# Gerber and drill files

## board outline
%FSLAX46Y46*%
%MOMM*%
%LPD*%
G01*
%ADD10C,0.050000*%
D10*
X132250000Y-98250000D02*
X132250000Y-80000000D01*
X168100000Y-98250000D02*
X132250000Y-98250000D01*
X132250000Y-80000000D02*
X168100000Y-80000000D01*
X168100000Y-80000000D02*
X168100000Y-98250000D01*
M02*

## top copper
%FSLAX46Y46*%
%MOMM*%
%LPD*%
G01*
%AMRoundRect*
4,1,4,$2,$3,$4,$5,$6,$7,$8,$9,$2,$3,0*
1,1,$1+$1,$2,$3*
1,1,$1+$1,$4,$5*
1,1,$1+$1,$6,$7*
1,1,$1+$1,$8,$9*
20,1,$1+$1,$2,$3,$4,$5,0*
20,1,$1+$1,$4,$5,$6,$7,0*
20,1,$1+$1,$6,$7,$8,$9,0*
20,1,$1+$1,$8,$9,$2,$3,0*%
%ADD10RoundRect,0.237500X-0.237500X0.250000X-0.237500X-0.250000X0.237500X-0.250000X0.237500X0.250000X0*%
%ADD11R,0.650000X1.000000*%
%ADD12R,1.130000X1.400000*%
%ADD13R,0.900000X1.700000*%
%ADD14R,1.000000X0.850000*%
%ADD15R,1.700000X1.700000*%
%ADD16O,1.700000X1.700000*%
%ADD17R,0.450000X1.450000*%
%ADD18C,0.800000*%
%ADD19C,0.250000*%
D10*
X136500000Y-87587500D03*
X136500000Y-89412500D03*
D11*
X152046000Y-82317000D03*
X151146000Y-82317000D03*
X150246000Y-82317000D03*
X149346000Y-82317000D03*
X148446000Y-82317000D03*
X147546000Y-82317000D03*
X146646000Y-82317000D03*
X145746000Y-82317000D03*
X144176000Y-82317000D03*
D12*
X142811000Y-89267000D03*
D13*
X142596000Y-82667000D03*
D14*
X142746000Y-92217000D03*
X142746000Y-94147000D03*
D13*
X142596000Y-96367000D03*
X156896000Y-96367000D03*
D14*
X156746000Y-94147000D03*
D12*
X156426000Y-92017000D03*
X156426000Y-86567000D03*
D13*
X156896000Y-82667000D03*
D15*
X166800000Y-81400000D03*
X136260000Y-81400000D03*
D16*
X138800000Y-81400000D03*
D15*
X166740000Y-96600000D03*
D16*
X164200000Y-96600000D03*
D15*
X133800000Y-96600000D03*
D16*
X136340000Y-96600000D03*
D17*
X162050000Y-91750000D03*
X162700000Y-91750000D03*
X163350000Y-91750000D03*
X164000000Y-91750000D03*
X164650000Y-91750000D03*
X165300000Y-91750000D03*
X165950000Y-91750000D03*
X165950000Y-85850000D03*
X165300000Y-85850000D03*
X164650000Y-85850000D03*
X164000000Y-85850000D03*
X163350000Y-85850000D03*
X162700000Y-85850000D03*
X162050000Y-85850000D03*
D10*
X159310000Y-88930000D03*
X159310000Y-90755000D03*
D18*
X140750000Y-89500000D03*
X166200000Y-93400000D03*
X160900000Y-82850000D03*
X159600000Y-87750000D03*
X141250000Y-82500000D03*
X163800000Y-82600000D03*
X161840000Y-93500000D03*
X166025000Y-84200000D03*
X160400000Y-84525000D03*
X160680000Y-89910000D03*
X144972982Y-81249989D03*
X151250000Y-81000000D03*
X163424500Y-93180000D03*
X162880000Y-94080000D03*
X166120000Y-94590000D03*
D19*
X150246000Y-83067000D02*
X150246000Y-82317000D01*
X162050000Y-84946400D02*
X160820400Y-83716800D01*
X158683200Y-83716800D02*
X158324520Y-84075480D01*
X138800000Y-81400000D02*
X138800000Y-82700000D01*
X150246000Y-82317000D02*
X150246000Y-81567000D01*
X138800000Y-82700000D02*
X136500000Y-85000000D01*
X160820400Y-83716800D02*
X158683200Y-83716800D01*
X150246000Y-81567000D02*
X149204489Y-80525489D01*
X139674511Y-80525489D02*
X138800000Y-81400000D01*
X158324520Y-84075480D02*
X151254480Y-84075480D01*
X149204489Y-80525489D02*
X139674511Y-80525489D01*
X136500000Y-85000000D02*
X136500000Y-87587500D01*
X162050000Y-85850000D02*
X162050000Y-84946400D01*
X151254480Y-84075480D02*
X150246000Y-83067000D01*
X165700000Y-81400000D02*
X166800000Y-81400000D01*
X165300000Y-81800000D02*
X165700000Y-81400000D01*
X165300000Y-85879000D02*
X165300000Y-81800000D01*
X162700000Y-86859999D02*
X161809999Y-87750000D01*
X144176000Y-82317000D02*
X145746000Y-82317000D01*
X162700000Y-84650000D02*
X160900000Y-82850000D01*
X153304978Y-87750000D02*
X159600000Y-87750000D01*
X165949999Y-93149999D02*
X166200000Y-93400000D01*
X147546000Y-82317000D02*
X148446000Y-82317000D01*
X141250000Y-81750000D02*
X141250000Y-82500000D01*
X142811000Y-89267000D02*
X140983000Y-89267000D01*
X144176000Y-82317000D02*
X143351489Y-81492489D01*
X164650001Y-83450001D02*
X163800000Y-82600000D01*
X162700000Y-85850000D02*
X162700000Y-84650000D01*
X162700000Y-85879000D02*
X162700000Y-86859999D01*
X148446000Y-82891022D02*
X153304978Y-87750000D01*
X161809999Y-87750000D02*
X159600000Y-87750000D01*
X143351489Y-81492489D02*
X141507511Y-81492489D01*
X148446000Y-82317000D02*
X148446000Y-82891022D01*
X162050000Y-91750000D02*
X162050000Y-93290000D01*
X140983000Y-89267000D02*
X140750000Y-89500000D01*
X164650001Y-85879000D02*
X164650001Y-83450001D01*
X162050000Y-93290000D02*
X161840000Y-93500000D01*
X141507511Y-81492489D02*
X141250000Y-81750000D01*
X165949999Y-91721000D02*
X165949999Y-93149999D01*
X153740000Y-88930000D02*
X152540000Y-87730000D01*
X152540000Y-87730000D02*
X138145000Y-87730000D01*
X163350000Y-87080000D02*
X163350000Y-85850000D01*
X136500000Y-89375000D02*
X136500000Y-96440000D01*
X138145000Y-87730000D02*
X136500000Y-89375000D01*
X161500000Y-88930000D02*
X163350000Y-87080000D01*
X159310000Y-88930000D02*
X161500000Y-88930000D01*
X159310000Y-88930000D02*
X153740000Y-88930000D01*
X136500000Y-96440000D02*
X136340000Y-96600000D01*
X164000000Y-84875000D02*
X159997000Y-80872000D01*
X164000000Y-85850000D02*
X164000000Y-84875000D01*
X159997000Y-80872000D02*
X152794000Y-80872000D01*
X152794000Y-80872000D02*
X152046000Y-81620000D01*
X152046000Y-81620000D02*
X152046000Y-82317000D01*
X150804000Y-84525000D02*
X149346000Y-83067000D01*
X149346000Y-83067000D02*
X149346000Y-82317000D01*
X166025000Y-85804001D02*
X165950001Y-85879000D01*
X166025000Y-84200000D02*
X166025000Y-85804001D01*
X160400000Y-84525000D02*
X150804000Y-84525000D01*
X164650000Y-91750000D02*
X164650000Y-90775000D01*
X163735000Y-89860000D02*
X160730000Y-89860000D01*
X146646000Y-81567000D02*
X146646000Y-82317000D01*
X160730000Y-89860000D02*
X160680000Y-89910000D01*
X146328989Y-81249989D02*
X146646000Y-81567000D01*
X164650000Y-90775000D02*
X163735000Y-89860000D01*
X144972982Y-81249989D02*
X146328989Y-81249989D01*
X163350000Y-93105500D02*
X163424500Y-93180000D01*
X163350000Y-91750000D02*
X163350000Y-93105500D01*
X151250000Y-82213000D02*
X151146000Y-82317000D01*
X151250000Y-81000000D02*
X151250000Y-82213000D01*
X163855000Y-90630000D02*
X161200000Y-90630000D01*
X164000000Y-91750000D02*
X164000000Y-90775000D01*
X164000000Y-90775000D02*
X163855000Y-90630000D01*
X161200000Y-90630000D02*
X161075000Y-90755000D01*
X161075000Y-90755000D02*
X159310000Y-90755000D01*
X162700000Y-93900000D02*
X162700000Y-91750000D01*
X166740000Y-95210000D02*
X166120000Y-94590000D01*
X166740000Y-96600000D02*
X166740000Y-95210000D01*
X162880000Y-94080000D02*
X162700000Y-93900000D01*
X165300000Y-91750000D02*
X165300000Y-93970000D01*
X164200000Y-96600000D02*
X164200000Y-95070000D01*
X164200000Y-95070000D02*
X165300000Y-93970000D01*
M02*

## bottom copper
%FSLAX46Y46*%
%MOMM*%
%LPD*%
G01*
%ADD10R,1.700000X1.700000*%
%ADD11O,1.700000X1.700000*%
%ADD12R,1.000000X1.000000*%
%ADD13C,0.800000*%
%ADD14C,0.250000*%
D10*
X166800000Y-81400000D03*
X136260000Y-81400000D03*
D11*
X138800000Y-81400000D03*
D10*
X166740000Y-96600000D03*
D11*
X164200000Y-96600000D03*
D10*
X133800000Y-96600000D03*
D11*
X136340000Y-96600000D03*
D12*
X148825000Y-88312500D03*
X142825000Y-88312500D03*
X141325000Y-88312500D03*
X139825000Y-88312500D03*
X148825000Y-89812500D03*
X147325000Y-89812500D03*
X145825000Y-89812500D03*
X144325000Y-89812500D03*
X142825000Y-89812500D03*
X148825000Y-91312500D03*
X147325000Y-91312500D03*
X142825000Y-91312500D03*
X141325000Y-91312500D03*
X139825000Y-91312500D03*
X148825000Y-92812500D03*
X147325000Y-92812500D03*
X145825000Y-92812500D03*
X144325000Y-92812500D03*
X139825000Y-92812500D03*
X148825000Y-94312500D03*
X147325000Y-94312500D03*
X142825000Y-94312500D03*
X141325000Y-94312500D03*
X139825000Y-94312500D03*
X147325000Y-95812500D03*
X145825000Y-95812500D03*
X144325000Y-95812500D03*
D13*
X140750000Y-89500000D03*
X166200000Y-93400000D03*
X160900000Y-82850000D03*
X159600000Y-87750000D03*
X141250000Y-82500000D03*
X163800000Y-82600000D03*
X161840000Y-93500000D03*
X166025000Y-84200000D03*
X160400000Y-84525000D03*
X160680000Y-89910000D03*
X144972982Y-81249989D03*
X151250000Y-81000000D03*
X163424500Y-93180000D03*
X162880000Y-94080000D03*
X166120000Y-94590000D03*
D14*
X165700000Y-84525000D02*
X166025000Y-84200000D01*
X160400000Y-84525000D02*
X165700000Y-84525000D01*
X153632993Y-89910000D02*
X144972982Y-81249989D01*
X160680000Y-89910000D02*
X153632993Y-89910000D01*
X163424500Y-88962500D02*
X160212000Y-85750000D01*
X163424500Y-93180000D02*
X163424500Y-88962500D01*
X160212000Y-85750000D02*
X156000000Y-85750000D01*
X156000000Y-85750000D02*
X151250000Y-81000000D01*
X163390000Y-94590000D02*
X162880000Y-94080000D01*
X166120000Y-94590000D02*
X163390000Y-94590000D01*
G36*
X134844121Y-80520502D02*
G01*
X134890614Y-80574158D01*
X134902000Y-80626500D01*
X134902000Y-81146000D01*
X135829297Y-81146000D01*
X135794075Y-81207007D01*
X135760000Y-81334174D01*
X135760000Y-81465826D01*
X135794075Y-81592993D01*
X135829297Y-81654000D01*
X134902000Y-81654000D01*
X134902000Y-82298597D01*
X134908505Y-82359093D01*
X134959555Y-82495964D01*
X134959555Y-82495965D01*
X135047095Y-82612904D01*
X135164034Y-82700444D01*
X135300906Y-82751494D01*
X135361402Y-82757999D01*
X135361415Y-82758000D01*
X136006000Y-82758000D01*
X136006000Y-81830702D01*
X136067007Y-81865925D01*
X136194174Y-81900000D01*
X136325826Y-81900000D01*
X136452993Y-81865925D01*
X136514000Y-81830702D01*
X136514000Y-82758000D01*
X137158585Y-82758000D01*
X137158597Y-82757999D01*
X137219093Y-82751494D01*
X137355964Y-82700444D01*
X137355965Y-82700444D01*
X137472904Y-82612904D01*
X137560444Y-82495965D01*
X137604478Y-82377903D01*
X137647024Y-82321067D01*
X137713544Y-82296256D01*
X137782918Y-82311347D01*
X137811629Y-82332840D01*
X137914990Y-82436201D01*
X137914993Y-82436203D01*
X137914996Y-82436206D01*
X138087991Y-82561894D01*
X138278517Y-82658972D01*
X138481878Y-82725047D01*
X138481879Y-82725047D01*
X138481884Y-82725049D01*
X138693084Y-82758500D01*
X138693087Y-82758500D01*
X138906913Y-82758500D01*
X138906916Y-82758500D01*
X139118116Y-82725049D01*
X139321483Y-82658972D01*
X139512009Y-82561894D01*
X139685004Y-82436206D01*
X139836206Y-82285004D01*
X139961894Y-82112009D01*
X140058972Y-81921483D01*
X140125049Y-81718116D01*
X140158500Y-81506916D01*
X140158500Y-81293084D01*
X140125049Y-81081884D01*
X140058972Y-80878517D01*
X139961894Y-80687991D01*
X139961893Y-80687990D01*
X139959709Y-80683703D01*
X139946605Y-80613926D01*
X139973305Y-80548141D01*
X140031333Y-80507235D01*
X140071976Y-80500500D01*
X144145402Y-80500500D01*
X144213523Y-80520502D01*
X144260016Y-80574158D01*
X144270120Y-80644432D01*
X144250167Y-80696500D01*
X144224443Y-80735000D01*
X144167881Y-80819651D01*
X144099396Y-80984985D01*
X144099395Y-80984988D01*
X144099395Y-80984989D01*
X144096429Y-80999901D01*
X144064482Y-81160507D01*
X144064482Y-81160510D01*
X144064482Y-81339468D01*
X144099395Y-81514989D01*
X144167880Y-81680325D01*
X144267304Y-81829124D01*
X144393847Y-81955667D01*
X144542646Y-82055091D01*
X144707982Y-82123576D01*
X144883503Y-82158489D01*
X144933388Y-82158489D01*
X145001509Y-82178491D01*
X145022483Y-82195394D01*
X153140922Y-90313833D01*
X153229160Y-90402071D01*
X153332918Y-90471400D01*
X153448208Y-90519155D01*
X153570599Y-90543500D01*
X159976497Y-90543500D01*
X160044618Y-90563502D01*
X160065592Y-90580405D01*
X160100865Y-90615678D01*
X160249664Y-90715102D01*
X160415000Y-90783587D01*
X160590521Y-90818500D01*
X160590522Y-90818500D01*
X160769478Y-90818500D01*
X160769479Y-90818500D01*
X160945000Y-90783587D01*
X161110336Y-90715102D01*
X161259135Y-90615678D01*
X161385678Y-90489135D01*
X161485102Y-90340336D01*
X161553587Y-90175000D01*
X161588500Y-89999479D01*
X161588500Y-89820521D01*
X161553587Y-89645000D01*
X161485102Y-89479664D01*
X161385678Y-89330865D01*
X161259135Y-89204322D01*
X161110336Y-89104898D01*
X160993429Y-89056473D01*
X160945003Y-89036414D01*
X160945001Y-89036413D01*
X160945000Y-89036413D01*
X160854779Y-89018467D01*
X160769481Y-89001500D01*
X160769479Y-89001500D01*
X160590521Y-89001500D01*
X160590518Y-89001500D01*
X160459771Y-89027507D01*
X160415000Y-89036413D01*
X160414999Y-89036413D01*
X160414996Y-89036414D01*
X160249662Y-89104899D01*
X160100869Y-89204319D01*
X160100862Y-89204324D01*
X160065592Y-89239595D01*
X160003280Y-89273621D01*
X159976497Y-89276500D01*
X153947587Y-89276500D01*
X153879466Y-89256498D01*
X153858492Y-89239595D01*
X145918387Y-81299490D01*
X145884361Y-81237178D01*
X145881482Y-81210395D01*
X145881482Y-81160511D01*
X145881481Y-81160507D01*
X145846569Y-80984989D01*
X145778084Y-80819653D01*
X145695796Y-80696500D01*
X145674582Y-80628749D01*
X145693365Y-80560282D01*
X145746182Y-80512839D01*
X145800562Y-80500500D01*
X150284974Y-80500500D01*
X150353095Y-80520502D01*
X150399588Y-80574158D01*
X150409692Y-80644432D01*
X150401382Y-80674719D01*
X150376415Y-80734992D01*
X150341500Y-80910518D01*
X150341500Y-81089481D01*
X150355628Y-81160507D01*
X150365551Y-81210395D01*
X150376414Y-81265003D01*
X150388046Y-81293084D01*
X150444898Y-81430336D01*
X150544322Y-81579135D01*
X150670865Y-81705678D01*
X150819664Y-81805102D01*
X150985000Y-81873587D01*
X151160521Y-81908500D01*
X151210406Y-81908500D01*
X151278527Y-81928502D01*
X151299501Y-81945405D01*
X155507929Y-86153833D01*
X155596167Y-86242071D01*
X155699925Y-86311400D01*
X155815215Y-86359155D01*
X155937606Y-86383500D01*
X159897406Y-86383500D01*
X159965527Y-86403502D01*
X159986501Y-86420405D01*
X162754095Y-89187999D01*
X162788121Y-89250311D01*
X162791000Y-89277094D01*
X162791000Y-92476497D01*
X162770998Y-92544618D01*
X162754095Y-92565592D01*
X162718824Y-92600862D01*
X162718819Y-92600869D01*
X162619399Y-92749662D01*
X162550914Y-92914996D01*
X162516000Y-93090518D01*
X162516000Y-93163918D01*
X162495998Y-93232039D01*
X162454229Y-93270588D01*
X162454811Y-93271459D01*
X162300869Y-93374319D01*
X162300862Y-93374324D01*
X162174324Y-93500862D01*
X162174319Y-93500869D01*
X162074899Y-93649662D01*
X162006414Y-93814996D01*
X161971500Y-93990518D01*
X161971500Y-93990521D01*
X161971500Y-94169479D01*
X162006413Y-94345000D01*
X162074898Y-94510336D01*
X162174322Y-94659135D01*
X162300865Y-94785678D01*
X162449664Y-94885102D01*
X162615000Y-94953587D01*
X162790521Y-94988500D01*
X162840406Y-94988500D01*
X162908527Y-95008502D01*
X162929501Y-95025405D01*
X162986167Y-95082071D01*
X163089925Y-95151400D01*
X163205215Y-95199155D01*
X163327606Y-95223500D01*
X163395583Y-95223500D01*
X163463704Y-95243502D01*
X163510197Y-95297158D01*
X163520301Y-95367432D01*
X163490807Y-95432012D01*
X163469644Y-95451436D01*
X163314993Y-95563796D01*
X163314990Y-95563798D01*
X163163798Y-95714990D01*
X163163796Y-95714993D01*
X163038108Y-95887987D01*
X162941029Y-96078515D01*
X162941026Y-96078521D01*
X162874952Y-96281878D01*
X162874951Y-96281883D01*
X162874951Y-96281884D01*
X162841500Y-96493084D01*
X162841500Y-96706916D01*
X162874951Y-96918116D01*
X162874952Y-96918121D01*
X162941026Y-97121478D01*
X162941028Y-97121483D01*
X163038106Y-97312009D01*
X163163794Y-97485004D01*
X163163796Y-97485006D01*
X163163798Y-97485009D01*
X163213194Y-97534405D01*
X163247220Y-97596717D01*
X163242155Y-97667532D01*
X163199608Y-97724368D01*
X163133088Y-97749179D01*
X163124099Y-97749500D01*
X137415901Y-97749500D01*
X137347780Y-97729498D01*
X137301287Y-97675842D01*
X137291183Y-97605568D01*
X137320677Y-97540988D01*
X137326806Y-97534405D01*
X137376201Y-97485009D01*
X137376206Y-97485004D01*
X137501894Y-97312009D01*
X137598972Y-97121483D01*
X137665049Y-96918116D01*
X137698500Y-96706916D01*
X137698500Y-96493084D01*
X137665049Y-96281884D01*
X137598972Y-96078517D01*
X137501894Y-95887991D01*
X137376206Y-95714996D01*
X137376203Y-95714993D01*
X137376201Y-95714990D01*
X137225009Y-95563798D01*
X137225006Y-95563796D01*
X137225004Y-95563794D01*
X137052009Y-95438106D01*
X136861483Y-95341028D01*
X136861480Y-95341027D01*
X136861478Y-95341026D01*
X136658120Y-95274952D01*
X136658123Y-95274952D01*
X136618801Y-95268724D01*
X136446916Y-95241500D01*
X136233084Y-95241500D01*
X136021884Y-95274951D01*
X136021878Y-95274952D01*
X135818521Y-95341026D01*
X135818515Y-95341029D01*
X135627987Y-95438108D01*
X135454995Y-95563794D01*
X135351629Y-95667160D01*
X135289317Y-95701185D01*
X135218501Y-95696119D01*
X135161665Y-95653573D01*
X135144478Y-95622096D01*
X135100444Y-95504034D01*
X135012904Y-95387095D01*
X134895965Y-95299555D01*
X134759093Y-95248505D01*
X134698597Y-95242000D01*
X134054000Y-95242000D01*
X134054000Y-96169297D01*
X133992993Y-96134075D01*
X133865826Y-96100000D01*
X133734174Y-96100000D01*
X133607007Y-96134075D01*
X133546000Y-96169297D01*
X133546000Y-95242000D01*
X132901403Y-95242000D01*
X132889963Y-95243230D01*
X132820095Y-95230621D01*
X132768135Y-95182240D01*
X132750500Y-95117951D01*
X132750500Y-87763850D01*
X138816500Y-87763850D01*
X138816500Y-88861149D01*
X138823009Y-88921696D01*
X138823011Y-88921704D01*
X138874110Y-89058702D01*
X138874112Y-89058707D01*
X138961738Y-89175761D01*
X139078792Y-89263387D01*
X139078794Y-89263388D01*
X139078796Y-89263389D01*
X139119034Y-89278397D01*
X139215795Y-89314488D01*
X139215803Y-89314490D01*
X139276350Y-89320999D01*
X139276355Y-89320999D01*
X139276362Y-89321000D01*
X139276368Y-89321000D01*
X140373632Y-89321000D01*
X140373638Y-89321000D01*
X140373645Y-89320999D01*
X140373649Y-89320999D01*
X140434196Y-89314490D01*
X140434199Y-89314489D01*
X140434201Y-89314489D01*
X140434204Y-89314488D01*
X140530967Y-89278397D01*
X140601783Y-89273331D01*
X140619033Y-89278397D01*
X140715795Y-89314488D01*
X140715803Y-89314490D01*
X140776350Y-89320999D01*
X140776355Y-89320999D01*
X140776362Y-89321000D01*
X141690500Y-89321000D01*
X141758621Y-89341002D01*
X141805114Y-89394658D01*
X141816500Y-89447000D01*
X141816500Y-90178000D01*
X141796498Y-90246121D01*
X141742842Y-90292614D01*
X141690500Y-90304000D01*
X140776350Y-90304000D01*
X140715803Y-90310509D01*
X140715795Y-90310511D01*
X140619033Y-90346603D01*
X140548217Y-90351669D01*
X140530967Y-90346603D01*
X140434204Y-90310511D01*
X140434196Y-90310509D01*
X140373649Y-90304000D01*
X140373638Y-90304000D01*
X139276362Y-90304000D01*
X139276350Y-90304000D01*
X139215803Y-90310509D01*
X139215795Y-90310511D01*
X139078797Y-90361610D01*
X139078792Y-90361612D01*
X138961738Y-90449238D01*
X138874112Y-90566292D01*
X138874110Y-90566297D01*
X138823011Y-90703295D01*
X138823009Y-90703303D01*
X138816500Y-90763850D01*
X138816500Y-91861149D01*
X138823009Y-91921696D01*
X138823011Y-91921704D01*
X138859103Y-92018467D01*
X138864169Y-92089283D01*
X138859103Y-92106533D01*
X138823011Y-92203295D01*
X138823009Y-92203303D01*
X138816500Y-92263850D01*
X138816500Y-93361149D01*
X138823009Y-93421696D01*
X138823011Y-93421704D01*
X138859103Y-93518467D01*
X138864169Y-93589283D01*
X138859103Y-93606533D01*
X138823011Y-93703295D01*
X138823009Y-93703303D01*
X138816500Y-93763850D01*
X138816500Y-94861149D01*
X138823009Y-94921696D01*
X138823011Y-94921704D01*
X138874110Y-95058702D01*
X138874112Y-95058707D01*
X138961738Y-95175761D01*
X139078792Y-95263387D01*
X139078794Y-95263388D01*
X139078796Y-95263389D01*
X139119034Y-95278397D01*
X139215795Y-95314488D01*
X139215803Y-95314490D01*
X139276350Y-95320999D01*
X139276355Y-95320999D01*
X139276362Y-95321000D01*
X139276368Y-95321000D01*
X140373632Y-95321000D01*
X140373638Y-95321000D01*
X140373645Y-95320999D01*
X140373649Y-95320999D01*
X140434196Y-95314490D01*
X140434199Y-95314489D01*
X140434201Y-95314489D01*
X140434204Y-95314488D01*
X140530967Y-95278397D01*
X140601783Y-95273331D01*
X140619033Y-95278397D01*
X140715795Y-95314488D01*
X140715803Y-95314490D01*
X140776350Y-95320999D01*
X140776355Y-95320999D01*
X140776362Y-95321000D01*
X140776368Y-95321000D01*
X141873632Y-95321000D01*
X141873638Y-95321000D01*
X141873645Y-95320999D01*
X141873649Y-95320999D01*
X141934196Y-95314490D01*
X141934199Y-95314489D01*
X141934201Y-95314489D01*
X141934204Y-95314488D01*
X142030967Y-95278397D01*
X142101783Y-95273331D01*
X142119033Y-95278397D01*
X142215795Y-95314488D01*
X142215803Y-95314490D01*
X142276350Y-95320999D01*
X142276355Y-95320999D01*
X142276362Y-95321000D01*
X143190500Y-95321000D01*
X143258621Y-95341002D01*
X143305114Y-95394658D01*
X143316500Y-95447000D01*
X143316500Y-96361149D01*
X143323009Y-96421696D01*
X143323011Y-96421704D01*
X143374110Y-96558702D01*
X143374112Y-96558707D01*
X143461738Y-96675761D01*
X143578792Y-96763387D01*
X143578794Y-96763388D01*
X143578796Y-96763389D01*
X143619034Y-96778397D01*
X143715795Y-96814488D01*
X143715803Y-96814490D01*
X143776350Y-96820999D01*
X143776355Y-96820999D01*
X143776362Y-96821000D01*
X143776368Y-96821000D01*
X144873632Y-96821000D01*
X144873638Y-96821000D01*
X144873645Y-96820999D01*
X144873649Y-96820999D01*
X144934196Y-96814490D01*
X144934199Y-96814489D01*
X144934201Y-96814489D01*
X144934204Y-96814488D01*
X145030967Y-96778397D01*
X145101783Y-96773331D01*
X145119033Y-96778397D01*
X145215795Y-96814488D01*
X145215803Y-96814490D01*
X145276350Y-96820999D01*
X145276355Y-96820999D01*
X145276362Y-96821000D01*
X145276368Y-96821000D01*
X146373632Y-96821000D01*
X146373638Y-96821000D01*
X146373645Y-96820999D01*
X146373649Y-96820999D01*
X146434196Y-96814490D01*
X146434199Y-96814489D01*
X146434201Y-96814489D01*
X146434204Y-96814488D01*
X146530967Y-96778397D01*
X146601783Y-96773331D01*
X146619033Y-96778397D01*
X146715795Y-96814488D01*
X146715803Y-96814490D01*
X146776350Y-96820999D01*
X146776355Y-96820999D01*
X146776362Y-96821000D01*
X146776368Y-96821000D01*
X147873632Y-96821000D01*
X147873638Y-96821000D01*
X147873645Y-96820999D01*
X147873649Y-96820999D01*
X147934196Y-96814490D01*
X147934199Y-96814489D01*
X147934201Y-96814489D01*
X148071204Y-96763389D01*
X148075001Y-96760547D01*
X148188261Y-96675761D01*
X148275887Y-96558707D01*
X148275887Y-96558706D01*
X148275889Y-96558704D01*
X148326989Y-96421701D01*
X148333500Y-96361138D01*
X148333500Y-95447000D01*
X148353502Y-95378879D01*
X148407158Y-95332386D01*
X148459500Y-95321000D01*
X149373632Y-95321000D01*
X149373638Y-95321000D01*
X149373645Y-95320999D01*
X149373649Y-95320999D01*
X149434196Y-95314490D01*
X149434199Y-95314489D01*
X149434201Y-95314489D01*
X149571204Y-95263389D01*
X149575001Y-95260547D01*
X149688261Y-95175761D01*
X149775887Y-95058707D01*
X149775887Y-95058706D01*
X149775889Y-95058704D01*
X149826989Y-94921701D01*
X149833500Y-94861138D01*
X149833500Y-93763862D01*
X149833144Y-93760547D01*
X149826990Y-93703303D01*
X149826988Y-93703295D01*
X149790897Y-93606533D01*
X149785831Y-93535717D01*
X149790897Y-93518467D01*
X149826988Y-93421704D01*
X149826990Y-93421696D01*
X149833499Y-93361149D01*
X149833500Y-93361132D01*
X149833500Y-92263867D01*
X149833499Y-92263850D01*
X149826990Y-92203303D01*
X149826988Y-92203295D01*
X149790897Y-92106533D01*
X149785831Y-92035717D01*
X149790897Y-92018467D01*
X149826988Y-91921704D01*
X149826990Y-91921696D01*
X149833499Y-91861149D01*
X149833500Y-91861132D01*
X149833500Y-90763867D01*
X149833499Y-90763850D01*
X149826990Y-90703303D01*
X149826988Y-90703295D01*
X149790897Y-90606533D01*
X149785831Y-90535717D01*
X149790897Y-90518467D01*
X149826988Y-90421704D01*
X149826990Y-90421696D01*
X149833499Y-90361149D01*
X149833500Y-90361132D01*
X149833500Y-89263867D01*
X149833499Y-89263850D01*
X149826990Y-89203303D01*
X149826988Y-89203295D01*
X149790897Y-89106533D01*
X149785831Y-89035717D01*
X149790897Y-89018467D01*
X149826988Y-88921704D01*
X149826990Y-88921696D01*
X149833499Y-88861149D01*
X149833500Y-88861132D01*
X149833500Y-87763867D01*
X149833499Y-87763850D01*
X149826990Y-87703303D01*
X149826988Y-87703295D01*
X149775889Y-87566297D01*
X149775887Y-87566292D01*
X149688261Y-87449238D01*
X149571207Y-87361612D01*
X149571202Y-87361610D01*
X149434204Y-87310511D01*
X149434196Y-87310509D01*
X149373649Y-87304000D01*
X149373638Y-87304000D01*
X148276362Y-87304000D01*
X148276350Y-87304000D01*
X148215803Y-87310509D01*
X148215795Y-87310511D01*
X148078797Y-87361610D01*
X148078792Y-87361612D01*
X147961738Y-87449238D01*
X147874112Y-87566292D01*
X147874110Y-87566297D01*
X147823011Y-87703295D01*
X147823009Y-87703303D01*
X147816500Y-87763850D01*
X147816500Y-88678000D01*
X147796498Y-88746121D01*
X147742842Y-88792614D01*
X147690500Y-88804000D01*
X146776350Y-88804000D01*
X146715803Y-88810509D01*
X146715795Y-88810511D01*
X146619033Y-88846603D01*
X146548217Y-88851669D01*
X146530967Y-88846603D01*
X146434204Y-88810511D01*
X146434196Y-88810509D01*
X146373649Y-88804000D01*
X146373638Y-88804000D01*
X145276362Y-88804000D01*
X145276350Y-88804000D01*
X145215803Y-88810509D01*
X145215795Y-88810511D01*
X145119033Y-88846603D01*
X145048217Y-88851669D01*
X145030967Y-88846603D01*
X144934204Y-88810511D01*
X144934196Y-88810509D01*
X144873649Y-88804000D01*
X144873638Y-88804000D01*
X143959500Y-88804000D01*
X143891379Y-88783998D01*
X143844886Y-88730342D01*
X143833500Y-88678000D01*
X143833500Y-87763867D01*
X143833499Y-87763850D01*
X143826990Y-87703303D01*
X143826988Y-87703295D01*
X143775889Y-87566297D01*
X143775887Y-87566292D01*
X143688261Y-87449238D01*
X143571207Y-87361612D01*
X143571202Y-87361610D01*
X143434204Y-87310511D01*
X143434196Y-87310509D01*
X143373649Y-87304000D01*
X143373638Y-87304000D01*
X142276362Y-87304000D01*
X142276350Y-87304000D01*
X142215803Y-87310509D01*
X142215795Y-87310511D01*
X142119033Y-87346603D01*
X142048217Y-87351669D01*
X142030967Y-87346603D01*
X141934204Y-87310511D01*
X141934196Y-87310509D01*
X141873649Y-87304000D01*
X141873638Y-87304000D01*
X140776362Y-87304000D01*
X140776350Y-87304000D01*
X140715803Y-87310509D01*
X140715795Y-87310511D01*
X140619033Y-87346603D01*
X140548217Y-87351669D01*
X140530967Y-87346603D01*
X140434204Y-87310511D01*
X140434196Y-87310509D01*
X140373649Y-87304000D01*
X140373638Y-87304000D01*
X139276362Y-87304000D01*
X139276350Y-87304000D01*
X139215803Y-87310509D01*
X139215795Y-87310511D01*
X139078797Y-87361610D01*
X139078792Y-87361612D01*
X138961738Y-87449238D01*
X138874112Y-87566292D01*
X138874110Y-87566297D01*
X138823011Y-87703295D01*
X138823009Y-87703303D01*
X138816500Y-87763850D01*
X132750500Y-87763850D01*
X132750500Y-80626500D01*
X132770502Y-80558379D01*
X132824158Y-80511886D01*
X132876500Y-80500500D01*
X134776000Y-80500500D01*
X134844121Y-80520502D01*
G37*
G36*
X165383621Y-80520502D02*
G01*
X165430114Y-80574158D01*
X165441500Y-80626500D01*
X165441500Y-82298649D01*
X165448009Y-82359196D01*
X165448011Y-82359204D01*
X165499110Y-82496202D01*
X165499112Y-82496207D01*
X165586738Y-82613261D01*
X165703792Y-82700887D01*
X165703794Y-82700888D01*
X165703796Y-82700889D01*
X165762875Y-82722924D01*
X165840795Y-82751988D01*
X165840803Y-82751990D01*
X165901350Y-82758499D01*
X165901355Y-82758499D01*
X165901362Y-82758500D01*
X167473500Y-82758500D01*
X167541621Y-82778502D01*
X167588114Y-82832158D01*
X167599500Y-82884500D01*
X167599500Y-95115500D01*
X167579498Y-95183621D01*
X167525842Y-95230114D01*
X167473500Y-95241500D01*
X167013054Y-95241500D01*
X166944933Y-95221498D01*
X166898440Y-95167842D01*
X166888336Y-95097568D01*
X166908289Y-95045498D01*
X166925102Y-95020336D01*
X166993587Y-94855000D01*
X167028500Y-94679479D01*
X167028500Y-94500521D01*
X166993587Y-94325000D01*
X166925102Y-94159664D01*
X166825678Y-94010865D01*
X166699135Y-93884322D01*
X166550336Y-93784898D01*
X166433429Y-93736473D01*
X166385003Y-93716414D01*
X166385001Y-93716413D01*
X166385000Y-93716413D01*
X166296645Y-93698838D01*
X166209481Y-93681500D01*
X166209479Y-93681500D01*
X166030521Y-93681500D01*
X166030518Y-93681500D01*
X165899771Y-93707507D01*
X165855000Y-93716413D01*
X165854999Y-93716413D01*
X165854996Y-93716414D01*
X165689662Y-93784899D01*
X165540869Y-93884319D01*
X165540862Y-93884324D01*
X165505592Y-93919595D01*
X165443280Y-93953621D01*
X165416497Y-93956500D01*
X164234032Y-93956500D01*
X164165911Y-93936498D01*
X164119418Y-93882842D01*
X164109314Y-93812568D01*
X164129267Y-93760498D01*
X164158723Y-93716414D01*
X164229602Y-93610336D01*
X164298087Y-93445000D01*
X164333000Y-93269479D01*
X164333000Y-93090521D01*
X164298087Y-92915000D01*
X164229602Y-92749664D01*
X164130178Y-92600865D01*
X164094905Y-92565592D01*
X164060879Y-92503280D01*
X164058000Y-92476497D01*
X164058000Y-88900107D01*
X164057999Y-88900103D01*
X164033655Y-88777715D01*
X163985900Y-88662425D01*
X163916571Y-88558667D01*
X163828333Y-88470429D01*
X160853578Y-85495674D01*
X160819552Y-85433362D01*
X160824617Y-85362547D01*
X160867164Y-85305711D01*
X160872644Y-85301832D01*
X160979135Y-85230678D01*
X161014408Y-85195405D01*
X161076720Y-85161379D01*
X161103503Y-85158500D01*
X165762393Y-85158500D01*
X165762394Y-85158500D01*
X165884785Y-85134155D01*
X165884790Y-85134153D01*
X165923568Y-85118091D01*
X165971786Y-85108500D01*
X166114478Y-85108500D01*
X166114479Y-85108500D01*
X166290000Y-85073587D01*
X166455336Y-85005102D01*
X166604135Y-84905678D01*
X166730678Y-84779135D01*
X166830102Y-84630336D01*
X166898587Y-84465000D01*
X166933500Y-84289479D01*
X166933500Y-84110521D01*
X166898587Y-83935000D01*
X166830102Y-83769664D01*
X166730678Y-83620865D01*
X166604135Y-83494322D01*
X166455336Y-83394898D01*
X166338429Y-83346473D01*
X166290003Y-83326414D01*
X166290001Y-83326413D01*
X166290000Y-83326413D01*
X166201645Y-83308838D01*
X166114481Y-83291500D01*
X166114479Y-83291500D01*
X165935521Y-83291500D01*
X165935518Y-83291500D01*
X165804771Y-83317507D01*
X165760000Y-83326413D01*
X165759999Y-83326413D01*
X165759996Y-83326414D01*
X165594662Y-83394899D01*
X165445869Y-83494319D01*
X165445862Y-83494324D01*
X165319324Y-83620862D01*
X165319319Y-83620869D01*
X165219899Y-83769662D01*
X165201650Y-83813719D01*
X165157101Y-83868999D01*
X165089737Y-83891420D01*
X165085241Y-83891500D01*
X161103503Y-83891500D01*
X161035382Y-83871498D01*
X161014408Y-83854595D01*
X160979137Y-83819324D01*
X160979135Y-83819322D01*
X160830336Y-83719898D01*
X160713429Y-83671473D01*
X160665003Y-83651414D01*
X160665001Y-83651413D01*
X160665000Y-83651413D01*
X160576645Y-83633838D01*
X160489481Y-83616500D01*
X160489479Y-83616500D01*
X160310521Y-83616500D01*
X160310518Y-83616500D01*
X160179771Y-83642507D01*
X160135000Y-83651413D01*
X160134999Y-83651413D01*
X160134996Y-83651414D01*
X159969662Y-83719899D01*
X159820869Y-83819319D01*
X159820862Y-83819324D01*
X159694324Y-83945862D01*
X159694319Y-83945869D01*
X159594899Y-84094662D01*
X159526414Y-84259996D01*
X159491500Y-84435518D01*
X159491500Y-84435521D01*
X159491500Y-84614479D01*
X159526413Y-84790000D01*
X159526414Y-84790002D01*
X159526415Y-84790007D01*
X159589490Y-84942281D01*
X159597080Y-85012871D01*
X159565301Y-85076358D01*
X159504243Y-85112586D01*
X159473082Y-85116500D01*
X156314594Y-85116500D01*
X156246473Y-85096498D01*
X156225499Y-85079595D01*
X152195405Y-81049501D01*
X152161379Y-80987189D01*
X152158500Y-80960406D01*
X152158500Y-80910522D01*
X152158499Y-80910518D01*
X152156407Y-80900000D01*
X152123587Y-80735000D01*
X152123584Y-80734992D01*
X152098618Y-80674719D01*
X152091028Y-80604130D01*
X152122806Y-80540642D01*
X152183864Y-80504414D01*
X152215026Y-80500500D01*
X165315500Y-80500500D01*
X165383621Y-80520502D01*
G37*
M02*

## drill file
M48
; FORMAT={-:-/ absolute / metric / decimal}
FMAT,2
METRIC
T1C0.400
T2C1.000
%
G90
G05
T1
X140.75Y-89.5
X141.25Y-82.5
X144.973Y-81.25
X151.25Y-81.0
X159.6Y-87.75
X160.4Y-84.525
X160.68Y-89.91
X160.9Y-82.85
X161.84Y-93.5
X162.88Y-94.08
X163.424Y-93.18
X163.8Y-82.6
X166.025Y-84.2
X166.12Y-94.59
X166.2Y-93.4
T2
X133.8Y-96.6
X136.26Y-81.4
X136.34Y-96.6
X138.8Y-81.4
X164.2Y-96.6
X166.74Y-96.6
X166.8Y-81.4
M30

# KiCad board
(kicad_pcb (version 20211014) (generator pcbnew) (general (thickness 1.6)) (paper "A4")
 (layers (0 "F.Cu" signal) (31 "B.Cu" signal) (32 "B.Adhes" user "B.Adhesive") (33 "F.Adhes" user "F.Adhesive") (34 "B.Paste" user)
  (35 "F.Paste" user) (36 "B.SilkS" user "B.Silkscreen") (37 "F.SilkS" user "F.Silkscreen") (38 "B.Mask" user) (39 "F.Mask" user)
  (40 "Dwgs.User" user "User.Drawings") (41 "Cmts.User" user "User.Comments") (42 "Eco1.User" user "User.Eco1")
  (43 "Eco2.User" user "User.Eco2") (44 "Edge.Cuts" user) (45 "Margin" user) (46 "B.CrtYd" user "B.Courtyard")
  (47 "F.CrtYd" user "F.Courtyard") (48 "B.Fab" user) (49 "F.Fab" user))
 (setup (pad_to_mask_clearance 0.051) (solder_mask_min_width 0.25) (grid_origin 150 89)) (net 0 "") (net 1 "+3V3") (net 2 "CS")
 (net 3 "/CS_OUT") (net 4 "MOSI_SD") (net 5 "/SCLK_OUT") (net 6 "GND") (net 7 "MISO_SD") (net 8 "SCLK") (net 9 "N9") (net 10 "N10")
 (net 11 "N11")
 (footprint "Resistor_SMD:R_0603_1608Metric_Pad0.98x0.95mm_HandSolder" (layer "F.Cu") (at 136.5 88.5 -90)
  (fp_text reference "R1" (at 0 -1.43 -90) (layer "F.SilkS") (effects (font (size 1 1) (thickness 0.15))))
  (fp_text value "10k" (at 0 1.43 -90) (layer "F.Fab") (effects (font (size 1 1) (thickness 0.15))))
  (pad "1" smd roundrect (at -0.9125 0 270) (size 0.975 0.95) (layers "F.Cu" "F.Paste" "F.Mask") (roundrect_rratio 0.25) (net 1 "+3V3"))
  (pad "2" smd roundrect (at 0.9125 0 270) (size 0.975 0.95) (layers "F.Cu" "F.Paste" "F.Mask") (roundrect_rratio 0.25) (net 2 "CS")))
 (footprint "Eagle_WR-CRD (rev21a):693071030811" (layer "F.Cu") (at 149.746 89.762)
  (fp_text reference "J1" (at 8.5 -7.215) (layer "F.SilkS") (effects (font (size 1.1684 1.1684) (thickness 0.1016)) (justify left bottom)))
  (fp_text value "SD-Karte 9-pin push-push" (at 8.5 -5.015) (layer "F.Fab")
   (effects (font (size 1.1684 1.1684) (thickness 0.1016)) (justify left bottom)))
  (pad "1" smd rect (at 2.3 -7.445) (size 0.65 1) (layers "F.Cu" "F.Paste" "F.Mask") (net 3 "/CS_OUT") (solder_mask_margin 0.1016))
  (pad "2" smd rect (at 1.4 -7.445) (size 0.65 1) (layers "F.Cu" "F.Paste" "F.Mask") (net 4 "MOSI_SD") (solder_mask_margin 0.1016))
  (pad "3" smd rect (at 0.5 -7.445) (size 0.65 1) (layers "F.Cu" "F.Paste" "F.Mask") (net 1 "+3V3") (solder_mask_margin 0.1016))
  (pad "4" smd rect (at -0.4 -7.445) (size 0.65 1) (layers "F.Cu" "F.Paste" "F.Mask") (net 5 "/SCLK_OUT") (solder_mask_margin 0.1016))
  (pad "5" smd rect (at -1.3 -7.445) (size 0.65 1) (layers "F.Cu" "F.Paste" "F.Mask") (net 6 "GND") (solder_mask_margin 0.1016))
  (pad "6" smd rect (at -2.2 -7.445) (size 0.65 1) (layers "F.Cu" "F.Paste" "F.Mask") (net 6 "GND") (solder_mask_margin 0.1016))
  (pad "7" smd rect (at -3.1 -7.445) (size 0.65 1) (layers "F.Cu" "F.Paste" "F.Mask") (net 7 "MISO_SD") (solder_mask_margin 0.1016))
  (pad "8" smd rect (at -4 -7.445) (size 0.65 1) (layers "F.Cu" "F.Paste" "F.Mask") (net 6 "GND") (solder_mask_margin 0.1016))
  (pad "9" smd rect (at -5.57 -7.445) (size 0.65 1) (layers "F.Cu" "F.Paste" "F.Mask") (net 6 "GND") (solder_mask_margin 0.1016))
  (pad "10" smd rect (at -6.935 -0.495) (size 1.13 1.4) (layers "F.Cu" "F.Paste" "F.Mask") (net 6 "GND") (solder_mask_margin 0.1016))
  (pad "11-1" smd rect (at -7.15 -7.095) (size 0.9 1.7) (layers "F.Cu" "F.Paste" "F.Mask") (solder_mask_margin 0.1016))
  (pad "11-3" smd rect (at -7 2.455) (size 1 0.85) (layers "F.Cu" "F.Paste" "F.Mask") (solder_mask_margin 0.1016))
  (pad "11-4" smd rect (at -7 4.385) (size 1 0.85) (layers "F.Cu" "F.Paste" "F.Mask") (solder_mask_margin 0.1016))
  (pad "11-5" smd rect (at -7.15 6.605) (size 0.9 1.7) (layers "F.Cu" "F.Paste" "F.Mask") (solder_mask_margin 0.1016))
  (pad "11-6" smd rect (at 7.15 6.605) (size 0.9 1.7) (layers "F.Cu" "F.Paste" "F.Mask") (solder_mask_margin 0.1016))
  (pad "11-7" smd rect (at 7 4.385 180) (size 1 0.85) (layers "F.Cu" "F.Paste" "F.Mask") (solder_mask_margin 0.1016))
  (pad "11-8" smd rect (at 6.68 2.255) (size 1.13 1.4) (layers "F.Cu" "F.Paste" "F.Mask") (solder_mask_margin 0.1016))
  (pad "11-9" smd rect (at 6.68 -3.195) (size 1.13 1.4) (layers "F.Cu" "F.Paste" "F.Mask") (solder_mask_margin 0.1016))
  (pad "11-10" smd rect (at 7.15 -7.095) (size 0.9 1.7) (layers "F.Cu" "F.Paste" "F.Mask") (solder_mask_margin 0.1016))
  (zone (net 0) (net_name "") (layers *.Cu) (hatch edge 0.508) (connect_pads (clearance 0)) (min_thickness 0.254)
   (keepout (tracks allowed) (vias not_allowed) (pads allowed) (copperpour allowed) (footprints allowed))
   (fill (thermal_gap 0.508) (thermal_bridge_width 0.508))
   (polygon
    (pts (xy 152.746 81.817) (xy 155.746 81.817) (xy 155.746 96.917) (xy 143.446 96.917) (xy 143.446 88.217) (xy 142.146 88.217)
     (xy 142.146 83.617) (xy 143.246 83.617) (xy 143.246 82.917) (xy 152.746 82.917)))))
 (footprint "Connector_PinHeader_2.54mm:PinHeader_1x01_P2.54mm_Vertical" (layer "F.Cu") (at 166.8 81.4)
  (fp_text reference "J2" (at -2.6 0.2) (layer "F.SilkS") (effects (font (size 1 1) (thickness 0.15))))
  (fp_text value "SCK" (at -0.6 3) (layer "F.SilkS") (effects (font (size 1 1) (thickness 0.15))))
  (pad "1" thru_hole rect locked (at 0 0) (size 1.7 1.7) (drill 1) (layers *.Cu *.Mask) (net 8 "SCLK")))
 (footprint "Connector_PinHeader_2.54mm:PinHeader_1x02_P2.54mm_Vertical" (layer "F.Cu") (at 136.26 81.4 90)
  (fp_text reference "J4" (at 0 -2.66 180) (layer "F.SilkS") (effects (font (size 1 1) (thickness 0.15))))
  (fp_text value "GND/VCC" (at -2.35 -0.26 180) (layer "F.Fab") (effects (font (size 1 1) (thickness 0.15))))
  (pad "1" thru_hole rect locked (at 0 0 90) (size 1.7 1.7) (drill 1) (layers *.Cu *.Mask) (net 6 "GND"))
  (pad "2" thru_hole oval locked (at 0 2.54 90) (size 1.7 1.7) (drill 1) (layers *.Cu *.Mask) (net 1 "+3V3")))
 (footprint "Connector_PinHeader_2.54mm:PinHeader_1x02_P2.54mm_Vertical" (layer "F.Cu") (at 166.74 96.6 -90)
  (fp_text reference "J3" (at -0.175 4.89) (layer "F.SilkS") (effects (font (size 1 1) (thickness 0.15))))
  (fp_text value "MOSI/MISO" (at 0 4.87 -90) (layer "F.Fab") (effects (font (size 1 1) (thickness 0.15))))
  (pad "1" thru_hole rect (at 0 0 270) (size 1.7 1.7) (drill 1) (layers *.Cu *.Mask) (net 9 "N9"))
  (pad "2" thru_hole oval (at 0 2.54 270) (size 1.7 1.7) (drill 1) (layers *.Cu *.Mask) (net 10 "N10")))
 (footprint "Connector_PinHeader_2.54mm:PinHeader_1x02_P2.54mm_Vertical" (layer "F.Cu") (at 133.8 96.6 90)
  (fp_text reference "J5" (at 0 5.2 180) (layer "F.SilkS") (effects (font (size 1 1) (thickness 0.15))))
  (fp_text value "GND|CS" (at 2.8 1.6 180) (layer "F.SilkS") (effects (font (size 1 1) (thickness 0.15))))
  (pad "1" thru_hole rect locked (at 0 0 90) (size 1.7 1.7) (drill 1) (layers *.Cu *.Mask) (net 6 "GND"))
  (pad "2" thru_hole oval locked (at 0 2.54 90) (size 1.7 1.7) (drill 1) (layers *.Cu *.Mask) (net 2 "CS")))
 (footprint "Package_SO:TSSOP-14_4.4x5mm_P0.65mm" (layer "F.Cu") (at 164 88.8 90)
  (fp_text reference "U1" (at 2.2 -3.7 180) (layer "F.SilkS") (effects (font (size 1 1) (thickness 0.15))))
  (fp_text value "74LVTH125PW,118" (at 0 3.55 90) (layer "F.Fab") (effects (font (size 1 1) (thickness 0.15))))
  (pad "1" smd rect locked (at -2.95 -1.95 90) (size 1.45 0.45) (layers "F.Cu" "F.Paste" "F.Mask") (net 6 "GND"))
  (pad "2" smd rect locked (at -2.95 -1.3 90) (size 1.45 0.45) (layers "F.Cu" "F.Paste" "F.Mask") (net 9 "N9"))
  (pad "3" smd rect locked (at -2.95 -0.65 90) (size 1.45 0.45) (layers "F.Cu" "F.Paste" "F.Mask") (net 4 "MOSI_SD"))
  (pad "4" smd rect locked (at -2.95 0 90) (size 1.45 0.45) (layers "F.Cu" "F.Paste" "F.Mask") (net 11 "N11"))
  (pad "5" smd rect locked (at -2.95 0.65 90) (size 1.45 0.45) (layers "F.Cu" "F.Paste" "F.Mask") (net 7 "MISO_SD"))
  (pad "6" smd rect locked (at -2.95 1.3 90) (size 1.45 0.45) (layers "F.Cu" "F.Paste" "F.Mask") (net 10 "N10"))
  (pad "7" smd rect locked (at -2.95 1.95 90) (size 1.45 0.45) (layers "F.Cu" "F.Paste" "F.Mask") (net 6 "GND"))
  (pad "8" smd rect locked (at 2.95 1.95 90) (size 1.45 0.45) (layers "F.Cu" "F.Paste" "F.Mask") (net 5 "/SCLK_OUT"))
  (pad "9" smd rect locked (at 2.95 1.3 90) (size 1.45 0.45) (layers "F.Cu" "F.Paste" "F.Mask") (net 8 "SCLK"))
  (pad "10" smd rect locked (at 2.95 0.65 90) (size 1.45 0.45) (layers "F.Cu" "F.Paste" "F.Mask") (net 6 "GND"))
  (pad "11" smd rect locked (at 2.95 0 90) (size 1.45 0.45) (layers "F.Cu" "F.Paste" "F.Mask") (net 3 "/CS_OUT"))
  (pad "12" smd rect locked (at 2.95 -0.65 90) (size 1.45 0.45) (layers "F.Cu" "F.Paste" "F.Mask") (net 2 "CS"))
  (pad "13" smd rect locked (at 2.95 -1.3 90) (size 1.45 0.45) (layers "F.Cu" "F.Paste" "F.Mask") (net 6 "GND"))
  (pad "14" smd rect locked (at 2.95 -1.95 90) (size 1.45 0.45) (layers "F.Cu" "F.Paste" "F.Mask") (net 1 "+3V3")))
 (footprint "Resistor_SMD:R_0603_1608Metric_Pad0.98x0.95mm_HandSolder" (layer "F.Cu") (at 159.31 89.8425 -90)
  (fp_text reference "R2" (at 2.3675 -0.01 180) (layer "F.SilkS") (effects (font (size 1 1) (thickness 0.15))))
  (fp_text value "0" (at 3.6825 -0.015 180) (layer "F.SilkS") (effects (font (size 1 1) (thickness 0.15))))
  (pad "1" smd roundrect (at -0.9125 0 270) (size 0.975 0.95) (layers "F.Cu" "F.Paste" "F.Mask") (roundrect_rratio 0.25) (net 2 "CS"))
  (pad "2" smd roundrect (at 0.9125 0 270) (size 0.975 0.95) (layers "F.Cu" "F.Paste" "F.Mask") (roundrect_rratio 0.25) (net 11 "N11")))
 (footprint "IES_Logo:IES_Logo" (layer "B.Cu") (at 146.325 85.8125 180)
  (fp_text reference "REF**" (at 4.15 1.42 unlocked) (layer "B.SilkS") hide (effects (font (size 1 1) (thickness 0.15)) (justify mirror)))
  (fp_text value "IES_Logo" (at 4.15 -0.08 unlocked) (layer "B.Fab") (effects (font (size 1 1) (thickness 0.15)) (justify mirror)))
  (pad "1" smd rect (at -2.5 -2.5 180) (size 1 1) (layers "B.Cu" "B.Paste" "B.Mask"))
  (pad "5" smd rect (at 3.5 -2.5 180) (size 1 1) (layers "B.Cu" "B.Paste" "B.Mask"))
  (pad "6" smd rect (at 5 -2.5 180) (size 1 1) (layers "B.Cu" "B.Paste" "B.Mask"))
  (pad "7" smd rect (at 6.5 -2.5 180) (size 1 1) (layers "B.Cu" "B.Paste" "B.Mask"))
  (pad "8" smd rect (at -2.5 -4 180) (size 1 1) (layers "B.Cu" "B.Paste" "B.Mask"))
  (pad "9" smd rect (at -1 -4 180) (size 1 1) (layers "B.Cu" "B.Paste" "B.Mask"))
  (pad "10" smd rect (at 0.5 -4 180) (size 1 1) (layers "B.Cu" "B.Paste" "B.Mask"))
  (pad "11" smd rect (at 2 -4 180) (size 1 1) (layers "B.Cu" "B.Paste" "B.Mask"))
  (pad "12" smd rect (at 3.5 -4 180) (size 1 1) (layers "B.Cu" "B.Paste" "B.Mask"))
  (pad "15" smd rect (at -2.5 -5.5 180) (size 1 1) (layers "B.Cu" "B.Paste" "B.Mask"))
  (pad "16" smd rect (at -1 -5.5 180) (size 1 1) (layers "B.Cu" "B.Paste" "B.Mask"))
  (pad "19" smd rect (at 3.5 -5.5 180) (size 1 1) (layers "B.Cu" "B.Paste" "B.Mask"))
  (pad "20" smd rect (at 5 -5.5 180) (size 1 1) (layers "B.Cu" "B.Paste" "B.Mask"))
  (pad "21" smd rect (at 6.5 -5.5 180) (size 1 1) (layers "B.Cu" "B.Paste" "B.Mask"))
  (pad "22" smd rect (at -2.5 -7 180) (size 1 1) (layers "B.Cu" "B.Paste" "B.Mask"))
  (pad "23" smd rect (at -1 -7 180) (size 1 1) (layers "B.Cu" "B.Paste" "B.Mask"))
  (pad "24" smd rect (at 0.5 -7 180) (size 1 1) (layers "B.Cu" "B.Paste" "B.Mask"))
  (pad "25" smd rect (at 2 -7 180) (size 1 1) (layers "B.Cu" "B.Paste" "B.Mask"))
  (pad "28" smd rect (at 6.5 -7 180) (size 1 1) (layers "B.Cu" "B.Paste" "B.Mask"))
  (pad "29" smd rect (at -2.5 -8.5 180) (size 1 1) (layers "B.Cu" "B.Paste" "B.Mask"))
  (pad "30" smd rect (at -1 -8.5 180) (size 1 1) (layers "B.Cu" "B.Paste" "B.Mask"))
  (pad "33" smd rect (at 3.5 -8.5 180) (size 1 1) (layers "B.Cu" "B.Paste" "B.Mask"))
  (pad "34" smd rect (at 5 -8.5 180) (size 1 1) (layers "B.Cu" "B.Paste" "B.Mask"))
  (pad "35" smd rect (at 6.5 -8.5 180) (size 1 1) (layers "B.Cu" "B.Paste" "B.Mask"))
  (pad "37" smd rect (at -1 -10 180) (size 1 1) (layers "B.Cu" "B.Paste" "B.Mask"))
  (pad "38" smd rect (at 0.5 -10 180) (size 1 1) (layers "B.Cu" "B.Paste" "B.Mask"))
  (pad "39" smd rect (at 2 -10 180) (size 1 1) (layers "B.Cu" "B.Paste" "B.Mask")))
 (gr_line (start 132.25 98.25) (end 132.25 80) (layer "Edge.Cuts") (width 0.05))
 (gr_line (start 168.1 98.25) (end 132.25 98.25) (layer "Edge.Cuts") (width 0.05))
 (gr_line (start 132.25 80) (end 168.1 80) (layer "Edge.Cuts") (width 0.05))
 (gr_line (start 168.1 80) (end 168.1 98.25) (layer "Edge.Cuts") (width 0.05))
 (segment (start 150.246 83.067) (end 150.246 82.317) (width 0.25) (layer "F.Cu") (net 1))
 (segment (start 162.05 84.9464) (end 160.8204 83.7168) (width 0.25) (layer "F.Cu") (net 1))
 (segment (start 158.6832 83.7168) (end 158.32452 84.07548) (width 0.25) (layer "F.Cu") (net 1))
 (segment (start 138.8 81.4) (end 138.8 82.7) (width 0.25) (layer "F.Cu") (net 1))
 (segment (start 150.246 82.317) (end 150.246 81.567) (width 0.25) (layer "F.Cu") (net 1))
 (segment (start 138.8 82.7) (end 136.5 85) (width 0.25) (layer "F.Cu") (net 1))
 (segment (start 160.8204 83.7168) (end 158.6832 83.7168) (width 0.25) (layer "F.Cu") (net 1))
 (segment (start 150.246 81.567) (end 149.204489 80.525489) (width 0.25) (layer "F.Cu") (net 1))
 (segment (start 139.674511 80.525489) (end 138.8 81.4) (width 0.25) (layer "F.Cu") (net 1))
 (segment (start 158.32452 84.07548) (end 151.25448 84.07548) (width 0.25) (layer "F.Cu") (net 1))
 (segment (start 149.204489 80.525489) (end 139.674511 80.525489) (width 0.25) (layer "F.Cu") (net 1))
 (segment (start 136.5 85) (end 136.5 87.5875) (width 0.25) (layer "F.Cu") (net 1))
 (segment (start 162.05 85.85) (end 162.05 84.9464) (width 0.25) (layer "F.Cu") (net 1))
 (segment (start 151.25448 84.07548) (end 150.246 83.067) (width 0.25) (layer "F.Cu") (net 1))
 (segment (start 165.7 81.4) (end 166.8 81.4) (width 0.25) (layer "F.Cu") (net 8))
 (segment (start 165.3 81.8) (end 165.7 81.4) (width 0.25) (layer "F.Cu") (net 8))
 (segment (start 165.3 85.879) (end 165.3 81.8) (width 0.25) (layer "F.Cu") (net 8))
 (segment (start 162.7 86.859999) (end 161.809999 87.75) (width 0.25) (layer "F.Cu") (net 6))
 (segment (start 144.176 82.317) (end 145.746 82.317) (width 0.25) (layer "F.Cu") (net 6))
 (segment (start 162.7 84.65) (end 160.9 82.85) (width 0.25) (layer "F.Cu") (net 6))
 (segment (start 153.304978 87.75) (end 159.6 87.75) (width 0.25) (layer "F.Cu") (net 6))
 (segment (start 165.949999 93.149999) (end 166.2 93.4) (width 0.25) (layer "F.Cu") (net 6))
 (segment (start 147.546 82.317) (end 148.446 82.317) (width 0.25) (layer "F.Cu") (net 6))
 (segment (start 141.25 81.75) (end 141.25 82.5) (width 0.25) (layer "F.Cu") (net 6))
 (segment (start 142.811 89.267) (end 140.983 89.267) (width 0.25) (layer "F.Cu") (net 6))
 (segment (start 144.176 82.317) (end 143.351489 81.492489) (width 0.25) (layer "F.Cu") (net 6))
 (segment (start 164.650001 83.450001) (end 163.8 82.6) (width 0.25) (layer "F.Cu") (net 6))
 (segment (start 162.7 85.85) (end 162.7 84.65) (width 0.25) (layer "F.Cu") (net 6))
 (segment (start 162.7 85.879) (end 162.7 86.859999) (width 0.25) (layer "F.Cu") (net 6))
 (segment (start 148.446 82.891022) (end 153.304978 87.75) (width 0.25) (layer "F.Cu") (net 6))
 (segment (start 161.809999 87.75) (end 159.6 87.75) (width 0.25) (layer "F.Cu") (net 6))
 (segment (start 143.351489 81.492489) (end 141.507511 81.492489) (width 0.25) (layer "F.Cu") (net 6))
 (segment (start 148.446 82.317) (end 148.446 82.891022) (width 0.25) (layer "F.Cu") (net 6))
 (segment (start 162.05 91.75) (end 162.05 93.29) (width 0.25) (layer "F.Cu") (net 6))
 (segment (start 140.983 89.267) (end 140.75 89.5) (width 0.25) (layer "F.Cu") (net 6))
 (segment (start 164.650001 85.879) (end 164.650001 83.450001) (width 0.25) (layer "F.Cu") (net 6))
 (segment (start 162.05 93.29) (end 161.84 93.5) (width 0.25) (layer "F.Cu") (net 6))
 (segment (start 141.507511 81.492489) (end 141.25 81.75) (width 0.25) (layer "F.Cu") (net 6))
 (segment (start 165.949999 91.721) (end 165.949999 93.149999) (width 0.25) (layer "F.Cu") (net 6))
 (via (at 140.75 89.5) (size 0.8) (drill 0.4) (layers "F.Cu" "B.Cu") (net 6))
 (via (at 166.2 93.4) (size 0.8) (drill 0.4) (layers "F.Cu" "B.Cu") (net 6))
 (via (at 160.9 82.85) (size 0.8) (drill 0.4) (layers "F.Cu" "B.Cu") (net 6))
 (via (at 159.6 87.75) (size 0.8) (drill 0.4) (layers "F.Cu" "B.Cu") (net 6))
 (via (at 141.25 82.5) (size 0.8) (drill 0.4) (layers "F.Cu" "B.Cu") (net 6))
 (via (at 163.8 82.6) (size 0.8) (drill 0.4) (layers "F.Cu" "B.Cu") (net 6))
 (via (at 161.84 93.5) (size 0.8) (drill 0.4) (layers "F.Cu" "B.Cu") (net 6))
 (segment (start 153.74 88.93) (end 152.54 87.73) (width 0.25) (layer "F.Cu") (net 2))
 (segment (start 152.54 87.73) (end 138.145 87.73) (width 0.25) (layer "F.Cu") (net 2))
 (segment (start 163.35 87.08) (end 163.35 85.85) (width 0.25) (layer "F.Cu") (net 2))
 (segment (start 136.5 89.375) (end 136.5 96.44) (width 0.25) (layer "F.Cu") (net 2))
 (segment (start 138.145 87.73) (end 136.5 89.375) (width 0.25) (layer "F.Cu") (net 2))
 (segment (start 161.5 88.93) (end 163.35 87.08) (width 0.25) (layer "F.Cu") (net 2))
 (segment (start 159.31 88.93) (end 161.5 88.93) (width 0.25) (layer "F.Cu") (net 2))
 (segment (start 159.31 88.93) (end 153.74 88.93) (width 0.25) (layer "F.Cu") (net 2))
 (segment (start 136.5 96.44) (end 136.34 96.6) (width 0.25) (layer "F.Cu") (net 2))
 (segment (start 164 84.875) (end 159.997 80.872) (width 0.25) (layer "F.Cu") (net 3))
 (segment (start 164 85.85) (end 164 84.875) (width 0.25) (layer "F.Cu") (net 3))
 (segment (start 159.997 80.872) (end 152.794 80.872) (width 0.25) (layer "F.Cu") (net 3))
 (segment (start 152.794 80.872) (end 152.046 81.62) (width 0.25) (layer "F.Cu") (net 3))
 (segment (start 152.046 81.62) (end 152.046 82.317) (width 0.25) (layer "F.Cu") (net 3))
 (segment (start 150.804 84.525) (end 149.346 83.067) (width 0.25) (layer "F.Cu") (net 5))
 (segment (start 149.346 83.067) (end 149.346 82.317) (width 0.25) (layer "F.Cu") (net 5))
 (segment (start 166.025 85.804001) (end 165.950001 85.879) (width 0.25) (layer "F.Cu") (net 5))
 (segment (start 166.025 84.2) (end 166.025 85.804001) (width 0.25) (layer "F.Cu") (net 5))
 (segment (start 160.4 84.525) (end 150.804 84.525) (width 0.25) (layer "F.Cu") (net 5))
 (via (at 166.025 84.2) (size 0.8) (drill 0.4) (layers "F.Cu" "B.Cu") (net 5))
 (via (at 160.4 84.525) (size 0.8) (drill 0.4) (layers "F.Cu" "B.Cu") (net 5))
 (segment (start 165.7 84.525) (end 166.025 84.2) (width 0.25) (layer "B.Cu") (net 5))
 (segment (start 160.4 84.525) (end 165.7 84.525) (width 0.25) (layer "B.Cu") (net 5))
 (segment (start 164.65 91.75) (end 164.65 90.775) (width 0.25) (layer "F.Cu") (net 7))
 (segment (start 163.735 89.86) (end 160.73 89.86) (width 0.25) (layer "F.Cu") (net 7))
 (segment (start 146.646 81.567) (end 146.646 82.317) (width 0.25) (layer "F.Cu") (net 7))
 (segment (start 160.73 89.86) (end 160.68 89.91) (width 0.25) (layer "F.Cu") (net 7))
 (segment (start 146.328989 81.249989) (end 146.646 81.567) (width 0.25) (layer "F.Cu") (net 7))
 (segment (start 164.65 90.775) (end 163.735 89.86) (width 0.25) (layer "F.Cu") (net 7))
 (segment (start 144.972982 81.249989) (end 146.328989 81.249989) (width 0.25) (layer "F.Cu") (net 7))
 (via (at 160.68 89.91) (size 0.8) (drill 0.4) (layers "F.Cu" "B.Cu") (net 7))
 (via (at 144.972982 81.249989) (size 0.8) (drill 0.4) (layers "F.Cu" "B.Cu") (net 7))
 (segment (start 153.632993 89.91) (end 144.972982 81.249989) (width 0.25) (layer "B.Cu") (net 7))
 (segment (start 160.68 89.91) (end 153.632993 89.91) (width 0.25) (layer "B.Cu") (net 7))
 (segment (start 163.35 93.1055) (end 163.4245 93.18) (width 0.25) (layer "F.Cu") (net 4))
 (segment (start 163.35 91.75) (end 163.35 93.1055) (width 0.25) (layer "F.Cu") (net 4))
 (segment (start 151.25 82.213) (end 151.146 82.317) (width 0.25) (layer "F.Cu") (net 4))
 (segment (start 151.25 81) (end 151.25 82.213) (width 0.25) (layer "F.Cu") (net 4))
 (via (at 151.25 81) (size 0.8) (drill 0.4) (layers "F.Cu" "B.Cu") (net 4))
 (via (at 163.4245 93.18) (size 0.8) (drill 0.4) (layers "F.Cu" "B.Cu") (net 4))
 (segment (start 163.4245 88.9625) (end 160.212 85.75) (width 0.25) (layer "B.Cu") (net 4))
 (segment (start 163.4245 93.18) (end 163.4245 88.9625) (width 0.25) (layer "B.Cu") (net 4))
 (segment (start 160.212 85.75) (end 156 85.75) (width 0.25) (layer "B.Cu") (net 4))
 (segment (start 156 85.75) (end 151.25 81) (width 0.25) (layer "B.Cu") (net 4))
 (segment (start 163.855 90.63) (end 161.2 90.63) (width 0.25) (layer "F.Cu") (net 11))
 (segment (start 164 91.75) (end 164 90.775) (width 0.25) (layer "F.Cu") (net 11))
 (segment (start 164 90.775) (end 163.855 90.63) (width 0.25) (layer "F.Cu") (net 11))
 (segment (start 161.2 90.63) (end 161.075 90.755) (width 0.25) (layer "F.Cu") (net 11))
 (segment (start 161.075 90.755) (end 159.31 90.755) (width 0.25) (layer "F.Cu") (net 11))
 (segment (start 162.7 93.9) (end 162.7 91.75) (width 0.25) (layer "F.Cu") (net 9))
 (segment (start 166.74 95.21) (end 166.12 94.59) (width 0.25) (layer "F.Cu") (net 9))
 (segment (start 166.74 96.6) (end 166.74 95.21) (width 0.25) (layer "F.Cu") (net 9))
 (segment (start 162.88 94.08) (end 162.7 93.9) (width 0.25) (layer "F.Cu") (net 9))
 (via (at 162.88 94.08) (size 0.8) (drill 0.4) (layers "F.Cu" "B.Cu") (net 9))
 (via (at 166.12 94.59) (size 0.8) (drill 0.4) (layers "F.Cu" "B.Cu") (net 9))
 (segment (start 163.39 94.59) (end 162.88 94.08) (width 0.25) (layer "B.Cu") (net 9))
 (segment (start 166.12 94.59) (end 163.39 94.59) (width 0.25) (layer "B.Cu") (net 9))
 (segment (start 165.3 91.75) (end 165.3 93.97) (width 0.25) (layer "F.Cu") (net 10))
 (segment (start 164.2 96.6) (end 164.2 95.07) (width 0.25) (layer "F.Cu") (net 10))
 (segment (start 164.2 95.07) (end 165.3 93.97) (width 0.25) (layer "F.Cu") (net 10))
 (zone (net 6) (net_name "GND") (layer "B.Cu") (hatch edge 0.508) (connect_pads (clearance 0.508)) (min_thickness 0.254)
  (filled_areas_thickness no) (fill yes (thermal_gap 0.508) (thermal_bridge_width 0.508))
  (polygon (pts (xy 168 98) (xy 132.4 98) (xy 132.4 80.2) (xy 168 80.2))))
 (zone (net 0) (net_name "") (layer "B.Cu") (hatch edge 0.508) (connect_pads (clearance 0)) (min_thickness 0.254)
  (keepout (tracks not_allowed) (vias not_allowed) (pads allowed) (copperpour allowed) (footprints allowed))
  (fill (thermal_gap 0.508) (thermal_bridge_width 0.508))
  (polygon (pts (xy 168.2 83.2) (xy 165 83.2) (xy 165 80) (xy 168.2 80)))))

